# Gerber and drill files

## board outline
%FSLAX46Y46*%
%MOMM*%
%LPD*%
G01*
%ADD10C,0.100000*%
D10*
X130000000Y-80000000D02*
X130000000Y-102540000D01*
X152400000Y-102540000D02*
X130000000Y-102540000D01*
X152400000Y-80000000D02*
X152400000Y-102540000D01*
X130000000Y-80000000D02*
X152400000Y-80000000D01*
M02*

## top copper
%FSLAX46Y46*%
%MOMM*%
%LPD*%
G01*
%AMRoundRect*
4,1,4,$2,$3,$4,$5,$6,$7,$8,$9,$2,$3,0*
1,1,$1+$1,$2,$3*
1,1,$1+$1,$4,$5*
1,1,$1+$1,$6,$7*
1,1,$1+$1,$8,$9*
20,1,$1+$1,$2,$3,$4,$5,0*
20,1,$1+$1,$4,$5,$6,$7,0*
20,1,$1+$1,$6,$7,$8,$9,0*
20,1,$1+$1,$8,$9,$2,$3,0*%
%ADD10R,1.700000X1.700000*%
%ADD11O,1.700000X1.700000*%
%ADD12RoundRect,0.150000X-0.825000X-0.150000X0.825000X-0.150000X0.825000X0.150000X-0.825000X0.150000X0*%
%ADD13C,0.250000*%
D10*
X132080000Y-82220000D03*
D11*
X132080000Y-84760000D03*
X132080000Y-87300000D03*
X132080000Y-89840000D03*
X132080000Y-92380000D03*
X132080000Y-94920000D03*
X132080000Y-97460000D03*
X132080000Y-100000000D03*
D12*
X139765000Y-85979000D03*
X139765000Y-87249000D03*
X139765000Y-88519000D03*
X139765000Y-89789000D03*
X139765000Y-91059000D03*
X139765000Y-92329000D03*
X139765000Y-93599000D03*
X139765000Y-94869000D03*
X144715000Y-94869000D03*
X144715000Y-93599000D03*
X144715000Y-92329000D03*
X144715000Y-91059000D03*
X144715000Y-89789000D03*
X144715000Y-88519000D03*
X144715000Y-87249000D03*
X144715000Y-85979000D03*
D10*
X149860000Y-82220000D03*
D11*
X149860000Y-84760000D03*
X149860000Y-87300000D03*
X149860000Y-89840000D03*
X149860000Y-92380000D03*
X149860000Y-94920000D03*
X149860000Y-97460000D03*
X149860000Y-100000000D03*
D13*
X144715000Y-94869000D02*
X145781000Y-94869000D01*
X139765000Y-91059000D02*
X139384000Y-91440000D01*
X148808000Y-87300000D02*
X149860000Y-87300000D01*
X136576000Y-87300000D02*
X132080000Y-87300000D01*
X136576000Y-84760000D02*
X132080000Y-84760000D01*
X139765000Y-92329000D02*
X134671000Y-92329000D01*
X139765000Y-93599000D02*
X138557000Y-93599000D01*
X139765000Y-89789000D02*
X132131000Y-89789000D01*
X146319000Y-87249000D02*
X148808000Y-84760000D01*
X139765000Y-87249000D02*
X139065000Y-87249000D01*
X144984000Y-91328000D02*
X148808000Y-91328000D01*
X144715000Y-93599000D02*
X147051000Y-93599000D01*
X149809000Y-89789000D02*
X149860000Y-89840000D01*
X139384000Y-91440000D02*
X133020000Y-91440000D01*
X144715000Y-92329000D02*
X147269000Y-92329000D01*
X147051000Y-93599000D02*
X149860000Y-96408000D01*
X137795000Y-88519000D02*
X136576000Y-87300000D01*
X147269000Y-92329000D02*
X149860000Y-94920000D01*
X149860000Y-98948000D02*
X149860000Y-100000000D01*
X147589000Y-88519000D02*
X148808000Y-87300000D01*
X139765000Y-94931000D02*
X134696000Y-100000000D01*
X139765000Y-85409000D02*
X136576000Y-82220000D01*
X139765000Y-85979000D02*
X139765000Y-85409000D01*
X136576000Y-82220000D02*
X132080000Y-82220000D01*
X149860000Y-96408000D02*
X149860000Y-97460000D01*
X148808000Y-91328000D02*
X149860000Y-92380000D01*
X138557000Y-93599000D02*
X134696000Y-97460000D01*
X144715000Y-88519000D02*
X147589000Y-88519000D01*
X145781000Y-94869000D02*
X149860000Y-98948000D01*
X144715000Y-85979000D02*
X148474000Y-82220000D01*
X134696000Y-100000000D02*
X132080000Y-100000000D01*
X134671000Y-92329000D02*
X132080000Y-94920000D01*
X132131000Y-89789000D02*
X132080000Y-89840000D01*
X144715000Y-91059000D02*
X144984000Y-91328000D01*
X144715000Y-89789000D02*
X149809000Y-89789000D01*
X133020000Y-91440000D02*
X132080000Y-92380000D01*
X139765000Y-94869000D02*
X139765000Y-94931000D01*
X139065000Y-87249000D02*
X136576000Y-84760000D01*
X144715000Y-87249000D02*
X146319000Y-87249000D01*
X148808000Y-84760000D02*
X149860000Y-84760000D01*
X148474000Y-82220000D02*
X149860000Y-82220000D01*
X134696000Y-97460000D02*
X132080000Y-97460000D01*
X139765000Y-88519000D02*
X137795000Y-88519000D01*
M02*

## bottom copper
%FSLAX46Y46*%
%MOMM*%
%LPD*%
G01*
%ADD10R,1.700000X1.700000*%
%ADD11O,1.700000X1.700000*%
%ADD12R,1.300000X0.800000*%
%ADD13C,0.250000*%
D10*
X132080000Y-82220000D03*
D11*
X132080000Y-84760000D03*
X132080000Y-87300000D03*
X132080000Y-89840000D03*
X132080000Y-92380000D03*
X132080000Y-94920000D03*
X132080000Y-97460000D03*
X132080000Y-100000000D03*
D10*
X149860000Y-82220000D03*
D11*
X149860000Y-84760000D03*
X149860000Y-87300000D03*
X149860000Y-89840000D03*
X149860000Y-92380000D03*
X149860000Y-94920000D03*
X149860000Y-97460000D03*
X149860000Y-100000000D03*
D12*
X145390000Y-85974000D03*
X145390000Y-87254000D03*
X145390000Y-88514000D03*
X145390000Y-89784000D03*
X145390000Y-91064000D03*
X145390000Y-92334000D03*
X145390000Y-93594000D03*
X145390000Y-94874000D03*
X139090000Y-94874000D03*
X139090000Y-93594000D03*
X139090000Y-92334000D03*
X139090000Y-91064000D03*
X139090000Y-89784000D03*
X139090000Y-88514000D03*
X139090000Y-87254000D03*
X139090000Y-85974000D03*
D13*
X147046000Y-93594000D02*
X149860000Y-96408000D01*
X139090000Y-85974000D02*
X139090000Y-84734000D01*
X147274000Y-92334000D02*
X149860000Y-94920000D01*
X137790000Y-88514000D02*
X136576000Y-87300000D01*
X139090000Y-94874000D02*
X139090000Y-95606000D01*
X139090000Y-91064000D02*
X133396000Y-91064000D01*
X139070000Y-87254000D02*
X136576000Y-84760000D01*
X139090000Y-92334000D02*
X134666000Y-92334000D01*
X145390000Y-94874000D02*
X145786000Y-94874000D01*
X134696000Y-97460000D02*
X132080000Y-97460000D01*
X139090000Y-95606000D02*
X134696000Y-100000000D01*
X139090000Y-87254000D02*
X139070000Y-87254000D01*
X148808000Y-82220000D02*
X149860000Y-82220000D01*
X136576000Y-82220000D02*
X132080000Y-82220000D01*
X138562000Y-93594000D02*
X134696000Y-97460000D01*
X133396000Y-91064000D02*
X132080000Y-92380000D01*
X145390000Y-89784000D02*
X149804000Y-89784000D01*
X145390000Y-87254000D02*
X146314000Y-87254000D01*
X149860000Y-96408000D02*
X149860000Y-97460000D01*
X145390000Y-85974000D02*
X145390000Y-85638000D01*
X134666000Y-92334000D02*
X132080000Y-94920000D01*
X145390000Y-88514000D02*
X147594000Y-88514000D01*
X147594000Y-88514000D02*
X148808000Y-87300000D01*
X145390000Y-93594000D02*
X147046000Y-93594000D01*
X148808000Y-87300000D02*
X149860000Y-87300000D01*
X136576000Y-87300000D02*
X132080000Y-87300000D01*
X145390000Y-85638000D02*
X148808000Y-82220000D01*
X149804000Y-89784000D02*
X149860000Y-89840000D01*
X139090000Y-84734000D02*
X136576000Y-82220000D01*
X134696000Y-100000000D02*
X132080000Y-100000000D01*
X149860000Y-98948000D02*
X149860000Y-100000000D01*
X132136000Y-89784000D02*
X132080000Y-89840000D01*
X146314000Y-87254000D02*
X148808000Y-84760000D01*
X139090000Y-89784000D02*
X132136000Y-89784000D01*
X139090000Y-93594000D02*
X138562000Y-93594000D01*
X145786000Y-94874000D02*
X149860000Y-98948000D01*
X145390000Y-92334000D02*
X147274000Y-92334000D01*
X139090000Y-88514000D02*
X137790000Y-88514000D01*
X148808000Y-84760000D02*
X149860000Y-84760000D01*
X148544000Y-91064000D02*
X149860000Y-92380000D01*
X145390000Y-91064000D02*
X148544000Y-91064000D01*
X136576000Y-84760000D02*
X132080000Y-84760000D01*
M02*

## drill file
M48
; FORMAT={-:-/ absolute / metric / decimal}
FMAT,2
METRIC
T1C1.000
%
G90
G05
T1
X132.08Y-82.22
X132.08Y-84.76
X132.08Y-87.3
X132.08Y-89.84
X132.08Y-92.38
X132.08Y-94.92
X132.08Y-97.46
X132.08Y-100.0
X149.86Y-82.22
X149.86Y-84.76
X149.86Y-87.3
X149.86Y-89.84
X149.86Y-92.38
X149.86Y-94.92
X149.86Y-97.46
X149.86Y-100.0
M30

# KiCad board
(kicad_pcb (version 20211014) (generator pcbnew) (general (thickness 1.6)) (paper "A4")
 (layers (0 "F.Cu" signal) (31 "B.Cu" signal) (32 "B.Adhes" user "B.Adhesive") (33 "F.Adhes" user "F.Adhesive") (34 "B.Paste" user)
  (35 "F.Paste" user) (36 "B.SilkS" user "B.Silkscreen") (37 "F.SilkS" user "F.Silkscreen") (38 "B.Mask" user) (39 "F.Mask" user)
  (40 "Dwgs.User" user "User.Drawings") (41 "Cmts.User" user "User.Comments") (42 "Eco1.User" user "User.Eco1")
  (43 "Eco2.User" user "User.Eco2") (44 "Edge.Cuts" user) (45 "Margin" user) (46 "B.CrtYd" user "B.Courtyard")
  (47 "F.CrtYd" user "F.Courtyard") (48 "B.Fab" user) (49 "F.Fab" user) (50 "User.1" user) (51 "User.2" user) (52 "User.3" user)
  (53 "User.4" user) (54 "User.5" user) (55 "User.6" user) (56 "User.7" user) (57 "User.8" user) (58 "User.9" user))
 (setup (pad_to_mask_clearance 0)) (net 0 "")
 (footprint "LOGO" (layer "F.Cu") (at 142.24 97.536)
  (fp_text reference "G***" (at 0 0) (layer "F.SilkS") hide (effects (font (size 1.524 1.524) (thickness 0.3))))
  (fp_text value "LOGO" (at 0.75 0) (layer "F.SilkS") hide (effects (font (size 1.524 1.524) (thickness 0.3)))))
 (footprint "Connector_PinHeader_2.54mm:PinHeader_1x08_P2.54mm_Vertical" (layer "F.Cu") (at 132.08 82.22)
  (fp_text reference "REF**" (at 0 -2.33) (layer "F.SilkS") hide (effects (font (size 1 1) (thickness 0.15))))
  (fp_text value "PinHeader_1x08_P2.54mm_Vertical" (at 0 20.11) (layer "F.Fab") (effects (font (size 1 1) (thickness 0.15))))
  (pad "1" thru_hole rect (at 0 0) (size 1.7 1.7) (drill 1) (layers *.Cu *.Mask))
  (pad "2" thru_hole oval (at 0 2.54) (size 1.7 1.7) (drill 1) (layers *.Cu *.Mask))
  (pad "3" thru_hole oval (at 0 5.08) (size 1.7 1.7) (drill 1) (layers *.Cu *.Mask))
  (pad "4" thru_hole oval (at 0 7.62) (size 1.7 1.7) (drill 1) (layers *.Cu *.Mask))
  (pad "5" thru_hole oval (at 0 10.16) (size 1.7 1.7) (drill 1) (layers *.Cu *.Mask))
  (pad "6" thru_hole oval (at 0 12.7) (size 1.7 1.7) (drill 1) (layers *.Cu *.Mask))
  (pad "7" thru_hole oval (at 0 15.24) (size 1.7 1.7) (drill 1) (layers *.Cu *.Mask))
  (pad "8" thru_hole oval (at 0 17.78) (size 1.7 1.7) (drill 1) (layers *.Cu *.Mask)))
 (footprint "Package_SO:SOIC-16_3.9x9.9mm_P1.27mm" (layer "F.Cu") (at 142.24 90.424)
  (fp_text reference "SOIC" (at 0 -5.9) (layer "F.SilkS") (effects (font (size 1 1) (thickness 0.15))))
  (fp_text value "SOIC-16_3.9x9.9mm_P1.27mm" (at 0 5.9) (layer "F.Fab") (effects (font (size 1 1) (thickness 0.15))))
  (pad "1" smd roundrect (at -2.475 -4.445) (size 1.95 0.6) (layers "F.Cu" "F.Paste" "F.Mask") (roundrect_rratio 0.25))
  (pad "2" smd roundrect (at -2.475 -3.175) (size 1.95 0.6) (layers "F.Cu" "F.Paste" "F.Mask") (roundrect_rratio 0.25))
  (pad "3" smd roundrect (at -2.475 -1.905) (size 1.95 0.6) (layers "F.Cu" "F.Paste" "F.Mask") (roundrect_rratio 0.25))
  (pad "4" smd roundrect (at -2.475 -0.635) (size 1.95 0.6) (layers "F.Cu" "F.Paste" "F.Mask") (roundrect_rratio 0.25))
  (pad "5" smd roundrect (at -2.475 0.635) (size 1.95 0.6) (layers "F.Cu" "F.Paste" "F.Mask") (roundrect_rratio 0.25))
  (pad "6" smd roundrect (at -2.475 1.905) (size 1.95 0.6) (layers "F.Cu" "F.Paste" "F.Mask") (roundrect_rratio 0.25))
  (pad "7" smd roundrect (at -2.475 3.175) (size 1.95 0.6) (layers "F.Cu" "F.Paste" "F.Mask") (roundrect_rratio 0.25))
  (pad "8" smd roundrect (at -2.475 4.445) (size 1.95 0.6) (layers "F.Cu" "F.Paste" "F.Mask") (roundrect_rratio 0.25))
  (pad "9" smd roundrect (at 2.475 4.445) (size 1.95 0.6) (layers "F.Cu" "F.Paste" "F.Mask") (roundrect_rratio 0.25))
  (pad "10" smd roundrect (at 2.475 3.175) (size 1.95 0.6) (layers "F.Cu" "F.Paste" "F.Mask") (roundrect_rratio 0.25))
  (pad "11" smd roundrect (at 2.475 1.905) (size 1.95 0.6) (layers "F.Cu" "F.Paste" "F.Mask") (roundrect_rratio 0.25))
  (pad "12" smd roundrect (at 2.475 0.635) (size 1.95 0.6) (layers "F.Cu" "F.Paste" "F.Mask") (roundrect_rratio 0.25))
  (pad "13" smd roundrect (at 2.475 -0.635) (size 1.95 0.6) (layers "F.Cu" "F.Paste" "F.Mask") (roundrect_rratio 0.25))
  (pad "14" smd roundrect (at 2.475 -1.905) (size 1.95 0.6) (layers "F.Cu" "F.Paste" "F.Mask") (roundrect_rratio 0.25))
  (pad "15" smd roundrect (at 2.475 -3.175) (size 1.95 0.6) (layers "F.Cu" "F.Paste" "F.Mask") (roundrect_rratio 0.25))
  (pad "16" smd roundrect (at 2.475 -4.445) (size 1.95 0.6) (layers "F.Cu" "F.Paste" "F.Mask") (roundrect_rratio 0.25)))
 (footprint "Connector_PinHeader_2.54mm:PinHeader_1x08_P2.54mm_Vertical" (layer "F.Cu") (at 149.86 82.22)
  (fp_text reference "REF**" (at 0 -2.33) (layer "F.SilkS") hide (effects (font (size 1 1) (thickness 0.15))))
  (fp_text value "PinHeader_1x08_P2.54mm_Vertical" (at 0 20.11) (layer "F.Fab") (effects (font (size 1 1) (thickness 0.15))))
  (pad "1" thru_hole rect (at 0 0) (size 1.7 1.7) (drill 1) (layers *.Cu *.Mask))
  (pad "2" thru_hole oval (at 0 2.54) (size 1.7 1.7) (drill 1) (layers *.Cu *.Mask))
  (pad "3" thru_hole oval (at 0 5.08) (size 1.7 1.7) (drill 1) (layers *.Cu *.Mask))
  (pad "4" thru_hole oval (at 0 7.62) (size 1.7 1.7) (drill 1) (layers *.Cu *.Mask))
  (pad "5" thru_hole oval (at 0 10.16) (size 1.7 1.7) (drill 1) (layers *.Cu *.Mask))
  (pad "6" thru_hole oval (at 0 12.7) (size 1.7 1.7) (drill 1) (layers *.Cu *.Mask))
  (pad "7" thru_hole oval (at 0 15.24) (size 1.7 1.7) (drill 1) (layers *.Cu *.Mask))
  (pad "8" thru_hole oval (at 0 17.78) (size 1.7 1.7) (drill 1) (layers *.Cu *.Mask)))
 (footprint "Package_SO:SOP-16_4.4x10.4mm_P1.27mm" (layer "B.Cu") (at 142.24 90.424 180)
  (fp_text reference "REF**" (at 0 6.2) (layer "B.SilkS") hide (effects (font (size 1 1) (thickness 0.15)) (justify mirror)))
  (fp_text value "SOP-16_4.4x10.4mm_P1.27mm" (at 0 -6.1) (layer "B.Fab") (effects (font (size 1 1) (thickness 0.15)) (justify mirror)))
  (pad "1" smd rect (at -3.15 4.45 180) (size 1.3 0.8) (layers "B.Cu" "B.Paste" "B.Mask"))
  (pad "2" smd rect (at -3.15 3.17 180) (size 1.3 0.8) (layers "B.Cu" "B.Paste" "B.Mask"))
  (pad "3" smd rect (at -3.15 1.91 180) (size 1.3 0.8) (layers "B.Cu" "B.Paste" "B.Mask"))
  (pad "4" smd rect (at -3.15 0.64 180) (size 1.3 0.8) (layers "B.Cu" "B.Paste" "B.Mask"))
  (pad "5" smd rect (at -3.15 -0.64 180) (size 1.3 0.8) (layers "B.Cu" "B.Paste" "B.Mask"))
  (pad "6" smd rect (at -3.15 -1.91 180) (size 1.3 0.8) (layers "B.Cu" "B.Paste" "B.Mask"))
  (pad "7" smd rect (at -3.15 -3.17 180) (size 1.3 0.8) (layers "B.Cu" "B.Paste" "B.Mask"))
  (pad "8" smd rect (at -3.15 -4.45 180) (size 1.3 0.8) (layers "B.Cu" "B.Paste" "B.Mask"))
  (pad "9" smd rect (at 3.15 -4.45 180) (size 1.3 0.8) (layers "B.Cu" "B.Paste" "B.Mask"))
  (pad "10" smd rect (at 3.15 -3.17 180) (size 1.3 0.8) (layers "B.Cu" "B.Paste" "B.Mask"))
  (pad "11" smd rect (at 3.15 -1.91 180) (size 1.3 0.8) (layers "B.Cu" "B.Paste" "B.Mask"))
  (pad "12" smd rect (at 3.15 -0.64 180) (size 1.3 0.8) (layers "B.Cu" "B.Paste" "B.Mask"))
  (pad "13" smd rect (at 3.15 0.64 180) (size 1.3 0.8) (layers "B.Cu" "B.Paste" "B.Mask"))
  (pad "14" smd rect (at 3.15 1.91 180) (size 1.3 0.8) (layers "B.Cu" "B.Paste" "B.Mask"))
  (pad "15" smd rect (at 3.15 3.17 180) (size 1.3 0.8) (layers "B.Cu" "B.Paste" "B.Mask"))
  (pad "16" smd rect (at 3.15 4.45 180) (size 1.3 0.8) (layers "B.Cu" "B.Paste" "B.Mask")))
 (gr_line (start 130 80) (end 130 102.54) (layer "Edge.Cuts") (width 0.1))
 (gr_line (start 152.4 102.54) (end 130 102.54) (layer "Edge.Cuts") (width 0.1))
 (gr_line (start 152.4 80) (end 152.4 102.54) (layer "Edge.Cuts") (width 0.1))
 (gr_line (start 130 80) (end 152.4 80) (layer "Edge.Cuts") (width 0.1))
 (segment (start 144.715 94.869) (end 145.781 94.869) (width 0.25) (layer "F.Cu") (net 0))
 (segment (start 139.765 91.059) (end 139.384 91.44) (width 0.25) (layer "F.Cu") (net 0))
 (segment (start 148.808 87.3) (end 149.86 87.3) (width 0.25) (layer "F.Cu") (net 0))
 (segment (start 136.576 87.3) (end 132.08 87.3) (width 0.25) (layer "F.Cu") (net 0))
 (segment (start 136.576 84.76) (end 132.08 84.76) (width 0.25) (layer "F.Cu") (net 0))
 (segment (start 139.765 92.329) (end 134.671 92.329) (width 0.25) (layer "F.Cu") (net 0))
 (segment (start 139.765 93.599) (end 138.557 93.599) (width 0.25) (layer "F.Cu") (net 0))
 (segment (start 139.765 89.789) (end 132.131 89.789) (width 0.25) (layer "F.Cu") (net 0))
 (segment (start 146.319 87.249) (end 148.808 84.76) (width 0.25) (layer "F.Cu") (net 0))
 (segment (start 139.765 87.249) (end 139.065 87.249) (width 0.25) (layer "F.Cu") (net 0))
 (segment (start 144.984 91.328) (end 148.808 91.328) (width 0.25) (layer "F.Cu") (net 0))
 (segment (start 144.715 93.599) (end 147.051 93.599) (width 0.25) (layer "F.Cu") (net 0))
 (segment (start 149.809 89.789) (end 149.86 89.84) (width 0.25) (layer "F.Cu") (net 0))
 (segment (start 139.384 91.44) (end 133.02 91.44) (width 0.25) (layer "F.Cu") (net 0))
 (segment (start 144.715 92.329) (end 147.269 92.329) (width 0.25) (layer "F.Cu") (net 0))
 (segment (start 147.051 93.599) (end 149.86 96.408) (width 0.25) (layer "F.Cu") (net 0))
 (segment (start 137.795 88.519) (end 136.576 87.3) (width 0.25) (layer "F.Cu") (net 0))
 (segment (start 147.269 92.329) (end 149.86 94.92) (width 0.25) (layer "F.Cu") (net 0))
 (segment (start 149.86 98.948) (end 149.86 100) (width 0.25) (layer "F.Cu") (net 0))
 (segment (start 147.589 88.519) (end 148.808 87.3) (width 0.25) (layer "F.Cu") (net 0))
 (segment (start 139.765 94.931) (end 134.696 100) (width 0.25) (layer "F.Cu") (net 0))
 (segment (start 139.765 85.409) (end 136.576 82.22) (width 0.25) (layer "F.Cu") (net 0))
 (segment (start 139.765 85.979) (end 139.765 85.409) (width 0.25) (layer "F.Cu") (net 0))
 (segment (start 136.576 82.22) (end 132.08 82.22) (width 0.25) (layer "F.Cu") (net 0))
 (segment (start 149.86 96.408) (end 149.86 97.46) (width 0.25) (layer "F.Cu") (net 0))
 (segment (start 148.808 91.328) (end 149.86 92.38) (width 0.25) (layer "F.Cu") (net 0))
 (segment (start 138.557 93.599) (end 134.696 97.46) (width 0.25) (layer "F.Cu") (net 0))
 (segment (start 144.715 88.519) (end 147.589 88.519) (width 0.25) (layer "F.Cu") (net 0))
 (segment (start 145.781 94.869) (end 149.86 98.948) (width 0.25) (layer "F.Cu") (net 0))
 (segment (start 144.715 85.979) (end 148.474 82.22) (width 0.25) (layer "F.Cu") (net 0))
 (segment (start 134.696 100) (end 132.08 100) (width 0.25) (layer "F.Cu") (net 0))
 (segment (start 134.671 92.329) (end 132.08 94.92) (width 0.25) (layer "F.Cu") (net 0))
 (segment (start 132.131 89.789) (end 132.08 89.84) (width 0.25) (layer "F.Cu") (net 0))
 (segment (start 144.715 91.059) (end 144.984 91.328) (width 0.25) (layer "F.Cu") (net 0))
 (segment (start 144.715 89.789) (end 149.809 89.789) (width 0.25) (layer "F.Cu") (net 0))
 (segment (start 133.02 91.44) (end 132.08 92.38) (width 0.25) (layer "F.Cu") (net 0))
 (segment (start 139.765 94.869) (end 139.765 94.931) (width 0.25) (layer "F.Cu") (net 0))
 (segment (start 139.065 87.249) (end 136.576 84.76) (width 0.25) (layer "F.Cu") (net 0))
 (segment (start 144.715 87.249) (end 146.319 87.249) (width 0.25) (layer "F.Cu") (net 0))
 (segment (start 148.808 84.76) (end 149.86 84.76) (width 0.25) (layer "F.Cu") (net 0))
 (segment (start 148.474 82.22) (end 149.86 82.22) (width 0.25) (layer "F.Cu") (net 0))
 (segment (start 134.696 97.46) (end 132.08 97.46) (width 0.25) (layer "F.Cu") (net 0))
 (segment (start 139.765 88.519) (end 137.795 88.519) (width 0.25) (layer "F.Cu") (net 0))
 (segment (start 147.046 93.594) (end 149.86 96.408) (width 0.25) (layer "B.Cu") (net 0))
 (segment (start 139.09 85.974) (end 139.09 84.734) (width 0.25) (layer "B.Cu") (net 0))
 (segment (start 147.274 92.334) (end 149.86 94.92) (width 0.25) (layer "B.Cu") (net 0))
 (segment (start 137.79 88.514) (end 136.576 87.3) (width 0.25) (layer "B.Cu") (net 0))
 (segment (start 139.09 94.874) (end 139.09 95.606) (width 0.25) (layer "B.Cu") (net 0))
 (segment (start 139.09 91.064) (end 133.396 91.064) (width 0.25) (layer "B.Cu") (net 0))
 (segment (start 139.07 87.254) (end 136.576 84.76) (width 0.25) (layer "B.Cu") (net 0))
 (segment (start 139.09 92.334) (end 134.666 92.334) (width 0.25) (layer "B.Cu") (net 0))
 (segment (start 145.39 94.874) (end 145.786 94.874) (width 0.25) (layer "B.Cu") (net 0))
 (segment (start 134.696 97.46) (end 132.08 97.46) (width 0.25) (layer "B.Cu") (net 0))
 (segment (start 139.09 95.606) (end 134.696 100) (width 0.25) (layer "B.Cu") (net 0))
 (segment (start 139.09 87.254) (end 139.07 87.254) (width 0.25) (layer "B.Cu") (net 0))
 (segment (start 148.808 82.22) (end 149.86 82.22) (width 0.25) (layer "B.Cu") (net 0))
 (segment (start 136.576 82.22) (end 132.08 82.22) (width 0.25) (layer "B.Cu") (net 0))
 (segment (start 138.562 93.594) (end 134.696 97.46) (width 0.25) (layer "B.Cu") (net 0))
 (segment (start 133.396 91.064) (end 132.08 92.38) (width 0.25) (layer "B.Cu") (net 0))
 (segment (start 145.39 89.784) (end 149.804 89.784) (width 0.25) (layer "B.Cu") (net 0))
 (segment (start 145.39 87.254) (end 146.314 87.254) (width 0.25) (layer "B.Cu") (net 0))
 (segment (start 149.86 96.408) (end 149.86 97.46) (width 0.25) (layer "B.Cu") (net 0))
 (segment (start 145.39 85.974) (end 145.39 85.638) (width 0.25) (layer "B.Cu") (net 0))
 (segment (start 134.666 92.334) (end 132.08 94.92) (width 0.25) (layer "B.Cu") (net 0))
 (segment (start 145.39 88.514) (end 147.594 88.514) (width 0.25) (layer "B.Cu") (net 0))
 (segment (start 147.594 88.514) (end 148.808 87.3) (width 0.25) (layer "B.Cu") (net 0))
 (segment (start 145.39 93.594) (end 147.046 93.594) (width 0.25) (layer "B.Cu") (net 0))
 (segment (start 148.808 87.3) (end 149.86 87.3) (width 0.25) (layer "B.Cu") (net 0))
 (segment (start 136.576 87.3) (end 132.08 87.3) (width 0.25) (layer "B.Cu") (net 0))
 (segment (start 145.39 85.638) (end 148.808 82.22) (width 0.25) (layer "B.Cu") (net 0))
 (segment (start 149.804 89.784) (end 149.86 89.84) (width 0.25) (layer "B.Cu") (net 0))
 (segment (start 139.09 84.734) (end 136.576 82.22) (width 0.25) (layer "B.Cu") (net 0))
 (segment (start 134.696 100) (end 132.08 100) (width 0.25) (layer "B.Cu") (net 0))
 (segment (start 149.86 98.948) (end 149.86 100) (width 0.25) (layer "B.Cu") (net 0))
 (segment (start 132.136 89.784) (end 132.08 89.84) (width 0.25) (layer "B.Cu") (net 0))
 (segment (start 146.314 87.254) (end 148.808 84.76) (width 0.25) (layer "B.Cu") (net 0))
 (segment (start 139.09 89.784) (end 132.136 89.784) (width 0.25) (layer "B.Cu") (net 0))
 (segment (start 139.09 93.594) (end 138.562 93.594) (width 0.25) (layer "B.Cu") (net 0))
 (segment (start 145.786 94.874) (end 149.86 98.948) (width 0.25) (layer "B.Cu") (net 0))
 (segment (start 145.39 92.334) (end 147.274 92.334) (width 0.25) (layer "B.Cu") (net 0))
 (segment (start 139.09 88.514) (end 137.79 88.514) (width 0.25) (layer "B.Cu") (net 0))
 (segment (start 148.808 84.76) (end 149.86 84.76) (width 0.25) (layer "B.Cu") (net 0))
 (segment (start 148.544 91.064) (end 149.86 92.38) (width 0.25) (layer "B.Cu") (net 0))
 (segment (start 145.39 91.064) (end 148.544 91.064) (width 0.25) (layer "B.Cu") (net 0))
 (segment (start 136.576 84.76) (end 132.08 84.76) (width 0.25) (layer "B.Cu") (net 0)))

